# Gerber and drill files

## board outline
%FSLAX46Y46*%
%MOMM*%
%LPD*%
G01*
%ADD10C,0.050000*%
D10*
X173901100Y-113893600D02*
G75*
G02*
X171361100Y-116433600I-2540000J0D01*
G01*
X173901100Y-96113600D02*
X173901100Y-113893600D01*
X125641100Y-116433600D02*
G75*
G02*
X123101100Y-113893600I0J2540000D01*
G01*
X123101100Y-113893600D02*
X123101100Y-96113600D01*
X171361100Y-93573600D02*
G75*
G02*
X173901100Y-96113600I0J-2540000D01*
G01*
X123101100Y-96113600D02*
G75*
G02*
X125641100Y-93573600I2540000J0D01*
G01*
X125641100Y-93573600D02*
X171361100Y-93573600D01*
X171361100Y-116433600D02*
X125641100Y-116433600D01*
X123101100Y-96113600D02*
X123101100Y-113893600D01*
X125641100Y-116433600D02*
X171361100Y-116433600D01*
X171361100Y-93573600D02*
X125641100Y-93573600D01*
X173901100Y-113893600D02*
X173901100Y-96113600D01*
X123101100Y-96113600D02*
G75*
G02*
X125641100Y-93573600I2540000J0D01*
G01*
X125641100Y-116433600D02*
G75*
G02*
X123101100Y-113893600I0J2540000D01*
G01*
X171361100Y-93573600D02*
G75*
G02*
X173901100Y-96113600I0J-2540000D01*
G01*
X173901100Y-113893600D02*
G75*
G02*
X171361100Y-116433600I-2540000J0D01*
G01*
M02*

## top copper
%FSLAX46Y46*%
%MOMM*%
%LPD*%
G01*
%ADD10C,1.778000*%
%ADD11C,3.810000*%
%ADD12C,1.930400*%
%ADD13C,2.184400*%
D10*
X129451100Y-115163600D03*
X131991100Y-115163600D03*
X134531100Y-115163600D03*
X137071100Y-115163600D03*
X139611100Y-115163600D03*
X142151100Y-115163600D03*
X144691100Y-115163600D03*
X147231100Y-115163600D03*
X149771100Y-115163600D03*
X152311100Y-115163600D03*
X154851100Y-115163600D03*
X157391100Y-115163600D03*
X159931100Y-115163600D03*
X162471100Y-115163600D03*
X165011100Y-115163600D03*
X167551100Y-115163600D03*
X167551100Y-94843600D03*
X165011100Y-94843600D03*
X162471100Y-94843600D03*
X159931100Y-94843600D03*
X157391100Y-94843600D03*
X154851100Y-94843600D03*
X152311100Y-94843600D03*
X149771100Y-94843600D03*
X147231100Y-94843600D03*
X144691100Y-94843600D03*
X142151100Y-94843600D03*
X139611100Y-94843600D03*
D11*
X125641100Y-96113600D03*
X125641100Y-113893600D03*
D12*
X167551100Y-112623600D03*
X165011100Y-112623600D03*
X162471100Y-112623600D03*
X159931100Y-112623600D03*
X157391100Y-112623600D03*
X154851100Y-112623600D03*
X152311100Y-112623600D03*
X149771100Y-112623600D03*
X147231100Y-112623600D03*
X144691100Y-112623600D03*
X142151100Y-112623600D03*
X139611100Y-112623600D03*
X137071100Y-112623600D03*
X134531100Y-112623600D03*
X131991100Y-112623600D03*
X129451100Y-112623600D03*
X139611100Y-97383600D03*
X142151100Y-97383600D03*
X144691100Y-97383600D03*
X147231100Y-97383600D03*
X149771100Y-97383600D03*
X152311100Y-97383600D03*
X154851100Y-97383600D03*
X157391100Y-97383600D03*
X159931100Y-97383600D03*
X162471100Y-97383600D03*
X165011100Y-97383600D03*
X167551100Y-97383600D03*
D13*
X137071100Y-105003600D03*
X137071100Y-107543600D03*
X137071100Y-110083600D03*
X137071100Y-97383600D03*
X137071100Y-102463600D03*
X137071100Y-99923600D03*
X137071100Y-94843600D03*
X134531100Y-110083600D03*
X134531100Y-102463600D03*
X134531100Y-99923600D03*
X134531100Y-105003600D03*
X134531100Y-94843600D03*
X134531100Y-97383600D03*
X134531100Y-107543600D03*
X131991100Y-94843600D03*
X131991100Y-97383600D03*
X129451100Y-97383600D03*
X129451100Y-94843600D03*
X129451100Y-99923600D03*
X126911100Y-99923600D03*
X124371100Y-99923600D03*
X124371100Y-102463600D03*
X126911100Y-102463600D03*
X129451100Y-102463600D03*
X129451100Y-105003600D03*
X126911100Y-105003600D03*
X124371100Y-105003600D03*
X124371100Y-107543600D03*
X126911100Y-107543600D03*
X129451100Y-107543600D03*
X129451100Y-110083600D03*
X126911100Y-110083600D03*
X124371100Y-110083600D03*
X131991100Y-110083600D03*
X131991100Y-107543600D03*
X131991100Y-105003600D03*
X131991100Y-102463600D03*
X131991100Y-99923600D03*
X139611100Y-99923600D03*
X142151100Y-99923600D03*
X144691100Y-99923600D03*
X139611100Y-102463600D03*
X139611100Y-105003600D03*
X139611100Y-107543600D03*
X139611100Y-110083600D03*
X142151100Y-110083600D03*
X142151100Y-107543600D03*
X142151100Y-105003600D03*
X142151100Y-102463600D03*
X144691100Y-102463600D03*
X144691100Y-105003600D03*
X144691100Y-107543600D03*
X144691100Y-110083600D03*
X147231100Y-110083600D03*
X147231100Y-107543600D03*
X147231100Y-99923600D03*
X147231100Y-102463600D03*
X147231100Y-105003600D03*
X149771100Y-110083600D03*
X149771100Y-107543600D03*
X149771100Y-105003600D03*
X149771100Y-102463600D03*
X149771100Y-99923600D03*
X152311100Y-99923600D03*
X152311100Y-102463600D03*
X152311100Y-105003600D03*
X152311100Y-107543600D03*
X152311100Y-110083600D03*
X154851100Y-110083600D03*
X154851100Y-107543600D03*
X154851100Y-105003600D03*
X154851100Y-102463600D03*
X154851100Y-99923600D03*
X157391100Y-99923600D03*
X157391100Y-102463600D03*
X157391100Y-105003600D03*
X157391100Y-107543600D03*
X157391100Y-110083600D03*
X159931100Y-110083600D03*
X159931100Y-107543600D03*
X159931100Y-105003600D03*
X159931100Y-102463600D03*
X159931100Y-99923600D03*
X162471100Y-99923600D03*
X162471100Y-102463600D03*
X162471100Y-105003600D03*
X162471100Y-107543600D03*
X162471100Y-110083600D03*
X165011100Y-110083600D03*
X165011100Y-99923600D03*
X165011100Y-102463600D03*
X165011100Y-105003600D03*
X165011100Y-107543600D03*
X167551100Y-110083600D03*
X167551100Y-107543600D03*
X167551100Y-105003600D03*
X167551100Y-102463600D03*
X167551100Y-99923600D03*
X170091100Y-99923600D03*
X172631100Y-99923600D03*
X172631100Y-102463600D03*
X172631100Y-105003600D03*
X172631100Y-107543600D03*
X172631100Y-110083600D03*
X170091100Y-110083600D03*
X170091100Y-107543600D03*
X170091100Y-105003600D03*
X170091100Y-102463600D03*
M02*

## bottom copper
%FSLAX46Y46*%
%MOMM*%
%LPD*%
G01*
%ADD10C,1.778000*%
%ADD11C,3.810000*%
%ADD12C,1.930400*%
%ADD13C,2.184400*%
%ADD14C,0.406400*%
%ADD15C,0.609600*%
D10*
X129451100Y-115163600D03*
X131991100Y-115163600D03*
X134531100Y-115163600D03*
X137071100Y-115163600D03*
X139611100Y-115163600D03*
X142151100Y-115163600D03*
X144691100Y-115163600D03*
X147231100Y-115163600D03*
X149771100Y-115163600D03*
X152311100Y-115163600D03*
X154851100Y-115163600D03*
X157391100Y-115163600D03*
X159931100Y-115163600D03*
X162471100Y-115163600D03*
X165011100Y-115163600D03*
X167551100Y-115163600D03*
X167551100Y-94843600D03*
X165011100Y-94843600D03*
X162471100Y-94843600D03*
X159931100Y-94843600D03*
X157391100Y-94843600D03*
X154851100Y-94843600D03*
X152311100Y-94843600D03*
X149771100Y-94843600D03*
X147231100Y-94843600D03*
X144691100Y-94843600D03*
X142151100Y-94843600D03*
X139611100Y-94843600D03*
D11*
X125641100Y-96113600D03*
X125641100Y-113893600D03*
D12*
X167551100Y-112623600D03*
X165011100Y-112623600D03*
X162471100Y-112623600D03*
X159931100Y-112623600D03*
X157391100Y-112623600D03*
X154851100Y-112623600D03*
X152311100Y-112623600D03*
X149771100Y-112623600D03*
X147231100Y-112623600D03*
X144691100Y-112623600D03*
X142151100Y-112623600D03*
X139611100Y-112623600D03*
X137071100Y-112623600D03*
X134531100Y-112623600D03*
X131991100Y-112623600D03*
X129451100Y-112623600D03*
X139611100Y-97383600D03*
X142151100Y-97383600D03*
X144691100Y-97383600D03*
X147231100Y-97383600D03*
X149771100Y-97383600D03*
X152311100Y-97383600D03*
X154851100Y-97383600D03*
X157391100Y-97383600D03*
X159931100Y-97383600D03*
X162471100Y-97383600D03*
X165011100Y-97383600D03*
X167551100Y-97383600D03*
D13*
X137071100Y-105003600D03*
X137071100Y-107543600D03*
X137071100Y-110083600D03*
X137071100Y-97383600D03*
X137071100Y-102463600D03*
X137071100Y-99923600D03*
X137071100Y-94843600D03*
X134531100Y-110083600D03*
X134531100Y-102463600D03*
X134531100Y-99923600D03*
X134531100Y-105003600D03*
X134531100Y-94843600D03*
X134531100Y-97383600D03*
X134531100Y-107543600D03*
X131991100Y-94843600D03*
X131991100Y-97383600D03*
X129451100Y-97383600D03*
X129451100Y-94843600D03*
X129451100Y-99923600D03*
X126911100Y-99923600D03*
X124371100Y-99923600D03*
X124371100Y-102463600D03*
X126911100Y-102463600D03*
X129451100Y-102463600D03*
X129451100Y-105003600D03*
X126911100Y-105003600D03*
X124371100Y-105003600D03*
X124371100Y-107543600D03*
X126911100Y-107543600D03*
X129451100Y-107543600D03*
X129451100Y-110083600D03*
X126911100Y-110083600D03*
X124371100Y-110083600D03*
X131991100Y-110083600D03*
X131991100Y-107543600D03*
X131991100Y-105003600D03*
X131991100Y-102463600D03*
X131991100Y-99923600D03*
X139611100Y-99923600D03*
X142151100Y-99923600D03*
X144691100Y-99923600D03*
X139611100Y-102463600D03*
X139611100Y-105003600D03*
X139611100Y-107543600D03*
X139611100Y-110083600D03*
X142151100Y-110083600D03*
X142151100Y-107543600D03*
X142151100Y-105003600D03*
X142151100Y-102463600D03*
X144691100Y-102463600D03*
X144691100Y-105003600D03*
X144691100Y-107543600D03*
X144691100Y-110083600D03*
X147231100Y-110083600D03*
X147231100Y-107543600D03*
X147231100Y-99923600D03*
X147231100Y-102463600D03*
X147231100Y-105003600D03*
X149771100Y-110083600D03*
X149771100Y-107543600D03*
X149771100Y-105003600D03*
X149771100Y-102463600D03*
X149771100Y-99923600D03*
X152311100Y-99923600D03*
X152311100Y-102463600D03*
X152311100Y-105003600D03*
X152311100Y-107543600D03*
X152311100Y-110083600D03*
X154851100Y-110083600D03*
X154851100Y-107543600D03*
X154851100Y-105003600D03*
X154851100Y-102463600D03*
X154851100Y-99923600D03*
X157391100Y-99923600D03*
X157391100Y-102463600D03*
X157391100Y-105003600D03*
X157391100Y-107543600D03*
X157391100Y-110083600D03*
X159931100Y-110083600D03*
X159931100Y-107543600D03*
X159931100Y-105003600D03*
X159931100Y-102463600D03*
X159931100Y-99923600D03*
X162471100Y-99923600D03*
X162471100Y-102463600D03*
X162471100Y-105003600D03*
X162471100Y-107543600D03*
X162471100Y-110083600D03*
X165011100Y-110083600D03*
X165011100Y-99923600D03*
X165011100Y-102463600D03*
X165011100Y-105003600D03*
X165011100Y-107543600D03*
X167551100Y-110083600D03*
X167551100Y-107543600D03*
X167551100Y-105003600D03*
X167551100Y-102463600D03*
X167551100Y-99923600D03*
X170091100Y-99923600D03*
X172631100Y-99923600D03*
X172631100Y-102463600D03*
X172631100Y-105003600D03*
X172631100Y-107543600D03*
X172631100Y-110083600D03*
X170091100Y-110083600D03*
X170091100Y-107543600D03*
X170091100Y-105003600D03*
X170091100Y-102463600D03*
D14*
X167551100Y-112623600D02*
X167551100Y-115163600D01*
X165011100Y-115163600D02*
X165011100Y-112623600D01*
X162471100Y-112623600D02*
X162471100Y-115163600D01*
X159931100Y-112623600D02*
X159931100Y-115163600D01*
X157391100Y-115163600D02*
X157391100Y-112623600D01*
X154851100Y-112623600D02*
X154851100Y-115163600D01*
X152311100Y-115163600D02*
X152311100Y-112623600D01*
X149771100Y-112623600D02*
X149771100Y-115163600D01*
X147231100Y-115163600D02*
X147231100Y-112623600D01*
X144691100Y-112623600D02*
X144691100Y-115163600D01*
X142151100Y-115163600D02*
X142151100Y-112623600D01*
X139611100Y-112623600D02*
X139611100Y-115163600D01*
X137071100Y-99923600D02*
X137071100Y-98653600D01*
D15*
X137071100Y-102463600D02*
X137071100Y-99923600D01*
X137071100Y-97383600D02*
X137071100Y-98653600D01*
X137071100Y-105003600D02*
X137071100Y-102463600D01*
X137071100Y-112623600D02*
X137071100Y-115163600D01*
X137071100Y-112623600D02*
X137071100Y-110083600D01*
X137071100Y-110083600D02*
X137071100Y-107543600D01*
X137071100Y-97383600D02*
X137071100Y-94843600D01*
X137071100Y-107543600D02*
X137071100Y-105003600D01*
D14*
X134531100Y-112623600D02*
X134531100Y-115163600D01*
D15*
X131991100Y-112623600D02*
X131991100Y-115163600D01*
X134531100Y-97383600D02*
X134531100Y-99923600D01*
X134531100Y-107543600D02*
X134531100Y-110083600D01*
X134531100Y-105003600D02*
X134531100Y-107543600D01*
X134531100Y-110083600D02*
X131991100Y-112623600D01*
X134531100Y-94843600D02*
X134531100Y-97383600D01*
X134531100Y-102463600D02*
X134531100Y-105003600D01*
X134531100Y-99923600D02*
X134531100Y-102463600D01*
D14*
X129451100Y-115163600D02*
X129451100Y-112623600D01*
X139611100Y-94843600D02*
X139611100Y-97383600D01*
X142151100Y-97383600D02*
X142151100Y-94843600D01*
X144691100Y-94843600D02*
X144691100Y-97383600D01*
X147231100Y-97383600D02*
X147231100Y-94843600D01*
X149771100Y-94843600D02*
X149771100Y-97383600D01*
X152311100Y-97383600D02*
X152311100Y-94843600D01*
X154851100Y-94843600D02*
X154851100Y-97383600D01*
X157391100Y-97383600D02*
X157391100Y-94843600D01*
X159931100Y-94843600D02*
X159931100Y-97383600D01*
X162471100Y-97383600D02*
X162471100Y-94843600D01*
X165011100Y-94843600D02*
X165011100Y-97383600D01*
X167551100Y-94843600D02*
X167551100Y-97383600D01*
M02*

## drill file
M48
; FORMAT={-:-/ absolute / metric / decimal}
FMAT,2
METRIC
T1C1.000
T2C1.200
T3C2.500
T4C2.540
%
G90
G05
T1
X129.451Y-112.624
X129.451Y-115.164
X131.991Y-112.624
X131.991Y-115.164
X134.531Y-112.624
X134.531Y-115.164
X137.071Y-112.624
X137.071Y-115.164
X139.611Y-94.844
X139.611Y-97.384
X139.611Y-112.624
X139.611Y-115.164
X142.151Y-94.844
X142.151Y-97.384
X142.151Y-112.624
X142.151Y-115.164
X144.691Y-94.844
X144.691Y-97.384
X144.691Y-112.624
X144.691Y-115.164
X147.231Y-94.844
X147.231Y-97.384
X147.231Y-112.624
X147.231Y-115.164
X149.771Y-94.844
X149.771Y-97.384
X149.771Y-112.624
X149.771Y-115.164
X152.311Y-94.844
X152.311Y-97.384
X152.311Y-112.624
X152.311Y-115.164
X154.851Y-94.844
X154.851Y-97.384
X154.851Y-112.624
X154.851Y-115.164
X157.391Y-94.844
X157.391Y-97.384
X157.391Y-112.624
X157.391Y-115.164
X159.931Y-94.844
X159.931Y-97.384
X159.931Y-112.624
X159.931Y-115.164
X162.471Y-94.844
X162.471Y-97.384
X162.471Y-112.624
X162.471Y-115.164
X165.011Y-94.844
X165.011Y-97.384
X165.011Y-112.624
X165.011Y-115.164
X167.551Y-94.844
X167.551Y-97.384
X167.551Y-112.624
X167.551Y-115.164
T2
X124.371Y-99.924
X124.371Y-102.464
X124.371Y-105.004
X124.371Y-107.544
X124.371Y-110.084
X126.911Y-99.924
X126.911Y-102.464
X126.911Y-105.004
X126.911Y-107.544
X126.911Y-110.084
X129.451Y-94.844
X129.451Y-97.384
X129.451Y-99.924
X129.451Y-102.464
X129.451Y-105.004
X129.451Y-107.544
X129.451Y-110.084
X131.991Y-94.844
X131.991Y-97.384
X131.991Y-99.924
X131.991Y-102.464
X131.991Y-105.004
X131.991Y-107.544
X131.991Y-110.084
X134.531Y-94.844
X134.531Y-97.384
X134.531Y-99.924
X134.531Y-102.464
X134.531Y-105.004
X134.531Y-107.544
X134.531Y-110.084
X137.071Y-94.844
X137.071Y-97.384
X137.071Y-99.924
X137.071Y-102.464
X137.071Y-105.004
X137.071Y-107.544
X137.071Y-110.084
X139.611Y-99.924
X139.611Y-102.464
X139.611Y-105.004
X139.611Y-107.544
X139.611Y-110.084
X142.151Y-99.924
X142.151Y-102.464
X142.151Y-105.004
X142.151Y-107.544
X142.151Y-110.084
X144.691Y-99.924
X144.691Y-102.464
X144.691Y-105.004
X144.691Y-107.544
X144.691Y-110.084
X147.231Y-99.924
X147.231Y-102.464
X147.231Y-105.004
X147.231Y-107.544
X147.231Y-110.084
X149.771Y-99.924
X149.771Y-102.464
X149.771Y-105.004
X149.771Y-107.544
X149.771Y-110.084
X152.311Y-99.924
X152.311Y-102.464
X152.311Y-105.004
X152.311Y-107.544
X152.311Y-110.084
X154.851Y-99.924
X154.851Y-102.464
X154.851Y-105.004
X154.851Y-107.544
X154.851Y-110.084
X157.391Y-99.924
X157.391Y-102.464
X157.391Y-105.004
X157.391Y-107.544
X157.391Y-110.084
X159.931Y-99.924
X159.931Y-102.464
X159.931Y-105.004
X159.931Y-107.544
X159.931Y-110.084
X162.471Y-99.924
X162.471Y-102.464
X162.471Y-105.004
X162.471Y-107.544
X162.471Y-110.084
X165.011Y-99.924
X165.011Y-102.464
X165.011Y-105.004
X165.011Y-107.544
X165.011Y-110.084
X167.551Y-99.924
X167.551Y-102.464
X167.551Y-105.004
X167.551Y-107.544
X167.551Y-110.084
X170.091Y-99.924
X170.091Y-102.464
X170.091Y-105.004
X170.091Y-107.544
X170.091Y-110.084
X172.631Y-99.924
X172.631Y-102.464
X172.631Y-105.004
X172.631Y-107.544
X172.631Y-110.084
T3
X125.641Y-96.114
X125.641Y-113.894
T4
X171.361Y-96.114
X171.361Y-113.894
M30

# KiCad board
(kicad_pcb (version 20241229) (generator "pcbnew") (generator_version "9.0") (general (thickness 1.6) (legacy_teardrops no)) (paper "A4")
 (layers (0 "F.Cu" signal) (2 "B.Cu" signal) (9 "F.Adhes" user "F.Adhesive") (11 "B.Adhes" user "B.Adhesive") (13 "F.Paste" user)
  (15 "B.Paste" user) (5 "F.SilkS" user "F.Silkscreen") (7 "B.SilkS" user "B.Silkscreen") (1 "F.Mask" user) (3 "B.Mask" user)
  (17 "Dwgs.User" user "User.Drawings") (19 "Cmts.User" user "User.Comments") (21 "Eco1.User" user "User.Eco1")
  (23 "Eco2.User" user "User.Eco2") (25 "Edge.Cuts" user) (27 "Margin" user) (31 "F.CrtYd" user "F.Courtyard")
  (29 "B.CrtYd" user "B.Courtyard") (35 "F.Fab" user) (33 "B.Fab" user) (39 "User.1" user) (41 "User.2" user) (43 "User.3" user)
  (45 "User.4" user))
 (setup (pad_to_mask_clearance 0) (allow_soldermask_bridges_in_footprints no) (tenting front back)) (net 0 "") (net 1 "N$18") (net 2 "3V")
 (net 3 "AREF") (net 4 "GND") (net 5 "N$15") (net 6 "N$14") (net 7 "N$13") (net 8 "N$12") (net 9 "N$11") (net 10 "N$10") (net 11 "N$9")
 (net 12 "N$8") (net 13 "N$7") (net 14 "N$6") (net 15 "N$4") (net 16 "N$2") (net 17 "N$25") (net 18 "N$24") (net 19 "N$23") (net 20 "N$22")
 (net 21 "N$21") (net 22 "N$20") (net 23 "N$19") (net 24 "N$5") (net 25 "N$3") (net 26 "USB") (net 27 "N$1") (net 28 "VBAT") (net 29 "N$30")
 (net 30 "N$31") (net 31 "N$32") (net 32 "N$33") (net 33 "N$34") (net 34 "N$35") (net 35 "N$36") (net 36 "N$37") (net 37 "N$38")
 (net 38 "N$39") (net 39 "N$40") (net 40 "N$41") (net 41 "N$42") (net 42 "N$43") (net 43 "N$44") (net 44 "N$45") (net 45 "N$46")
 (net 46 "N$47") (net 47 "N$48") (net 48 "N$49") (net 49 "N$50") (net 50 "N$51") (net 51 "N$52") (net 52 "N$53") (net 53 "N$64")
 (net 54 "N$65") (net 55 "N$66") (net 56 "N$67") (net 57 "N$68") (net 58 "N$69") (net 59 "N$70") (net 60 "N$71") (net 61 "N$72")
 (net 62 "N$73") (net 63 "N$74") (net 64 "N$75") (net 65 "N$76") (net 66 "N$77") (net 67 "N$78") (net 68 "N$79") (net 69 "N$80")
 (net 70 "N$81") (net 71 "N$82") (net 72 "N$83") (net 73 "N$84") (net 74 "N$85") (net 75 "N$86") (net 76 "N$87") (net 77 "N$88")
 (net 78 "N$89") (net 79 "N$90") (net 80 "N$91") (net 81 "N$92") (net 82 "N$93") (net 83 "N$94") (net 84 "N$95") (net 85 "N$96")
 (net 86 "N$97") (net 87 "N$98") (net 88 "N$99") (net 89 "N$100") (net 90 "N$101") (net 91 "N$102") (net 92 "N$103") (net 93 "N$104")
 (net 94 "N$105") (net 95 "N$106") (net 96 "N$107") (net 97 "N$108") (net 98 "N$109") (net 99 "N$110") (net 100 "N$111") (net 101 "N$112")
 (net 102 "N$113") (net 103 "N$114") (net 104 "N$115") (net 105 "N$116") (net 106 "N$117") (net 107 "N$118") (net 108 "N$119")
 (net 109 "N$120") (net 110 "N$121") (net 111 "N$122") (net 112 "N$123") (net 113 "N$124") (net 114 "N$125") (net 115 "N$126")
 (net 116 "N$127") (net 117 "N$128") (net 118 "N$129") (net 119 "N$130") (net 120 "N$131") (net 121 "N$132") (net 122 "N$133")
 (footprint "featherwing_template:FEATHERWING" (layer "F.Cu") (at 123.1011 116.4336)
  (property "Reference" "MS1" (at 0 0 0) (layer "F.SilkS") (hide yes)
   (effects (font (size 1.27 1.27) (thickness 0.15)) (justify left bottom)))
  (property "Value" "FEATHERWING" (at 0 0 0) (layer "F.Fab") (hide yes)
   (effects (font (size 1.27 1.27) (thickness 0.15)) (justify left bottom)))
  (fp_line (start 0 -20.32) (end 0 -2.54) (stroke (width 0.05) (type solid)) (layer "Edge.Cuts"))
  (fp_line (start 2.54 0) (end 48.26 0) (stroke (width 0.05) (type solid)) (layer "Edge.Cuts"))
  (fp_line (start 48.26 -22.86) (end 2.54 -22.86) (stroke (width 0.05) (type solid)) (layer "Edge.Cuts"))
  (fp_line (start 50.8 -2.54) (end 50.8 -20.32) (stroke (width 0.05) (type solid)) (layer "Edge.Cuts"))
  (fp_arc (start 0 -20.32) (mid 0.743949 -22.116051) (end 2.54 -22.86) (stroke (width 0.05) (type solid)) (layer "Edge.Cuts"))
  (fp_arc (start 2.54 0) (mid 0.743949 -0.743949) (end 0 -2.54) (stroke (width 0.05) (type solid)) (layer "Edge.Cuts"))
  (fp_arc (start 48.26 -22.86) (mid 50.056051 -22.116051) (end 50.8 -20.32) (stroke (width 0.05) (type solid)) (layer "Edge.Cuts"))
  (fp_arc (start 50.8 -2.54) (mid 50.056051 -0.743949) (end 48.26 0) (stroke (width 0.05) (type solid)) (layer "Edge.Cuts"))
  (pad "" np_thru_hole circle (at 48.26 -20.32) (size 2.54 2.54) (drill 2.54) (layers "*.Cu" "*.Mask"))
  (pad "" np_thru_hole circle (at 48.26 -2.54) (size 2.54 2.54) (drill 2.54) (layers "*.Cu" "*.Mask"))
  (pad "1" thru_hole circle (at 6.35 -1.27) (size 1.778 1.778) (drill 1) (layers "*.Cu" "*.Mask") (remove_unused_layers no) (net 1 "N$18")
   (solder_mask_margin 0.0508) (thermal_bridge_angle 0))
  (pad "2" thru_hole circle (at 8.89 -1.27) (size 1.778 1.778) (drill 1) (layers "*.Cu" "*.Mask") (remove_unused_layers no) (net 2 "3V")
   (solder_mask_margin 0.0508) (thermal_bridge_angle 0))
  (pad "3" thru_hole circle (at 11.43 -1.27) (size 1.778 1.778) (drill 1) (layers "*.Cu" "*.Mask") (remove_unused_layers no) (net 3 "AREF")
   (solder_mask_margin 0.0508) (thermal_bridge_angle 0))
  (pad "4" thru_hole circle (at 13.97 -1.27) (size 1.778 1.778) (drill 1) (layers "*.Cu" "*.Mask") (remove_unused_layers no) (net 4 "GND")
   (solder_mask_margin 0.0508) (thermal_bridge_angle 0))
  (pad "5" thru_hole circle (at 16.51 -1.27) (size 1.778 1.778) (drill 1) (layers "*.Cu" "*.Mask") (remove_unused_layers no) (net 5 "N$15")
   (solder_mask_margin 0.0508) (thermal_bridge_angle 0))
  (pad "6" thru_hole circle (at 19.05 -1.27) (size 1.778 1.778) (drill 1) (layers "*.Cu" "*.Mask") (remove_unused_layers no) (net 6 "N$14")
   (solder_mask_margin 0.0508) (thermal_bridge_angle 0))
  (pad "7" thru_hole circle (at 21.59 -1.27) (size 1.778 1.778) (drill 1) (layers "*.Cu" "*.Mask") (remove_unused_layers no) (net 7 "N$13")
   (solder_mask_margin 0.0508) (thermal_bridge_angle 0))
  (pad "8" thru_hole circle (at 24.13 -1.27) (size 1.778 1.778) (drill 1) (layers "*.Cu" "*.Mask") (remove_unused_layers no) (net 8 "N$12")
   (solder_mask_margin 0.0508) (thermal_bridge_angle 0))
  (pad "9" thru_hole circle (at 26.67 -1.27) (size 1.778 1.778) (drill 1) (layers "*.Cu" "*.Mask") (remove_unused_layers no) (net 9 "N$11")
   (solder_mask_margin 0.0508) (thermal_bridge_angle 0))
  (pad "10" thru_hole circle (at 29.21 -1.27) (size 1.778 1.778) (drill 1) (layers "*.Cu" "*.Mask") (remove_unused_layers no)
   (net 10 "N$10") (solder_mask_margin 0.0508) (thermal_bridge_angle 0))
  (pad "11" thru_hole circle (at 31.75 -1.27) (size 1.778 1.778) (drill 1) (layers "*.Cu" "*.Mask") (remove_unused_layers no) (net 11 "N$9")
   (solder_mask_margin 0.0508) (thermal_bridge_angle 0))
  (pad "12" thru_hole circle (at 34.29 -1.27) (size 1.778 1.778) (drill 1) (layers "*.Cu" "*.Mask") (remove_unused_layers no) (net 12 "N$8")
   (solder_mask_margin 0.0508) (thermal_bridge_angle 0))
  (pad "13" thru_hole circle (at 36.83 -1.27) (size 1.778 1.778) (drill 1) (layers "*.Cu" "*.Mask") (remove_unused_layers no) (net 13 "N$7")
   (solder_mask_margin 0.0508) (thermal_bridge_angle 0))
  (pad "14" thru_hole circle (at 39.37 -1.27) (size 1.778 1.778) (drill 1) (layers "*.Cu" "*.Mask") (remove_unused_layers no) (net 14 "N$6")
   (solder_mask_margin 0.0508) (thermal_bridge_angle 0))
  (pad "15" thru_hole circle (at 41.91 -1.27) (size 1.778 1.778) (drill 1) (layers "*.Cu" "*.Mask") (remove_unused_layers no) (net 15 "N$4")
   (solder_mask_margin 0.0508) (thermal_bridge_angle 0))
  (pad "16" thru_hole circle (at 44.45 -1.27) (size 1.778 1.778) (drill 1) (layers "*.Cu" "*.Mask") (remove_unused_layers no) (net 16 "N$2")
   (solder_mask_margin 0.0508) (thermal_bridge_angle 0))
  (pad "17" thru_hole circle (at 44.45 -21.59) (size 1.778 1.778) (drill 1) (layers "*.Cu" "*.Mask") (remove_unused_layers no)
   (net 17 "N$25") (solder_mask_margin 0.0508) (thermal_bridge_angle 0))
  (pad "18" thru_hole circle (at 41.91 -21.59) (size 1.778 1.778) (drill 1) (layers "*.Cu" "*.Mask") (remove_unused_layers no)
   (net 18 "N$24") (solder_mask_margin 0.0508) (thermal_bridge_angle 0))
  (pad "19" thru_hole circle (at 39.37 -21.59) (size 1.778 1.778) (drill 1) (layers "*.Cu" "*.Mask") (remove_unused_layers no)
   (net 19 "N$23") (solder_mask_margin 0.0508) (thermal_bridge_angle 0))
  (pad "20" thru_hole circle (at 36.83 -21.59) (size 1.778 1.778) (drill 1) (layers "*.Cu" "*.Mask") (remove_unused_layers no)
   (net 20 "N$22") (solder_mask_margin 0.0508) (thermal_bridge_angle 0))
  (pad "21" thru_hole circle (at 34.29 -21.59) (size 1.778 1.778) (drill 1) (layers "*.Cu" "*.Mask") (remove_unused_layers no)
   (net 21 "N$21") (solder_mask_margin 0.0508) (thermal_bridge_angle 0))
  (pad "22" thru_hole circle (at 31.75 -21.59) (size 1.778 1.778) (drill 1) (layers "*.Cu" "*.Mask") (remove_unused_layers no)
   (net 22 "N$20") (solder_mask_margin 0.0508) (thermal_bridge_angle 0))
  (pad "23" thru_hole circle (at 29.21 -21.59) (size 1.778 1.778) (drill 1) (layers "*.Cu" "*.Mask") (remove_unused_layers no)
   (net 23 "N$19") (solder_mask_margin 0.0508) (thermal_bridge_angle 0))
  (pad "24" thru_hole circle (at 26.67 -21.59) (size 1.778 1.778) (drill 1) (layers "*.Cu" "*.Mask") (remove_unused_layers no)
   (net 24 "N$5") (solder_mask_margin 0.0508) (thermal_bridge_angle 0))
  (pad "25" thru_hole circle (at 24.13 -21.59) (size 1.778 1.778) (drill 1) (layers "*.Cu" "*.Mask") (remove_unused_layers no)
   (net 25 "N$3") (solder_mask_margin 0.0508) (thermal_bridge_angle 0))
  (pad "26" thru_hole circle (at 21.59 -21.59) (size 1.778 1.778) (drill 1) (layers "*.Cu" "*.Mask") (remove_unused_layers no)
   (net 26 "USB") (solder_mask_margin 0.0508) (thermal_bridge_angle 0))
  (pad "27" thru_hole circle (at 19.05 -21.59) (size 1.778 1.778) (drill 1) (layers "*.Cu" "*.Mask") (remove_unused_layers no)
   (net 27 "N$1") (solder_mask_margin 0.0508) (thermal_bridge_angle 0))
  (pad "28" thru_hole circle (at 16.51 -21.59) (size 1.778 1.778) (drill 1) (layers "*.Cu" "*.Mask") (remove_unused_layers no)
   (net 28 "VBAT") (solder_mask_margin 0.0508) (thermal_bridge_angle 0))
  (pad "P$1" thru_hole circle (at 2.54 -20.32) (size 3.81 3.81) (drill 2.5) (layers "*.Cu" "*.Mask") (remove_unused_layers no)
   (solder_mask_margin 0.0508) (thermal_bridge_angle 0))
  (pad "P$2" thru_hole circle (at 2.54 -2.54) (size 3.81 3.81) (drill 2.5) (layers "*.Cu" "*.Mask") (remove_unused_layers no)
   (solder_mask_margin 0.0508) (thermal_bridge_angle 0)))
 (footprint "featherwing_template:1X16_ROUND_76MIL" (layer "F.Cu") (at 148.5011 112.6236 180)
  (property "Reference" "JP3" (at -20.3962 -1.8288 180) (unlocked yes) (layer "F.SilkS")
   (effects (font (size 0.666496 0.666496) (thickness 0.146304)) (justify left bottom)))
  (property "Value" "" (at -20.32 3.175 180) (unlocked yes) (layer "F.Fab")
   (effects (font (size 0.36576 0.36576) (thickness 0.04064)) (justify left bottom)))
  (pad "1" thru_hole circle (at -19.05 0 270) (size 1.9304 1.9304) (drill 1) (layers "*.Cu" "*.Mask") (remove_unused_layers no)
   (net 16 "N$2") (solder_mask_margin 0.0508) (thermal_bridge_angle 0))
  (pad "2" thru_hole circle (at -16.51 0 270) (size 1.9304 1.9304) (drill 1) (layers "*.Cu" "*.Mask") (remove_unused_layers no)
   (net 15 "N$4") (solder_mask_margin 0.0508) (thermal_bridge_angle 0))
  (pad "3" thru_hole circle (at -13.97 0 270) (size 1.9304 1.9304) (drill 1) (layers "*.Cu" "*.Mask") (remove_unused_layers no)
   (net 14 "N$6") (solder_mask_margin 0.0508) (thermal_bridge_angle 0))
  (pad "4" thru_hole circle (at -11.43 0 270) (size 1.9304 1.9304) (drill 1) (layers "*.Cu" "*.Mask") (remove_unused_layers no)
   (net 13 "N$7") (solder_mask_margin 0.0508) (thermal_bridge_angle 0))
  (pad "5" thru_hole circle (at -8.89 0 270) (size 1.9304 1.9304) (drill 1) (layers "*.Cu" "*.Mask") (remove_unused_layers no)
   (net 12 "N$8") (solder_mask_margin 0.0508) (thermal_bridge_angle 0))
  (pad "6" thru_hole circle (at -6.35 0 270) (size 1.9304 1.9304) (drill 1) (layers "*.Cu" "*.Mask") (remove_unused_layers no)
   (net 11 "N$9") (solder_mask_margin 0.0508) (thermal_bridge_angle 0))
  (pad "7" thru_hole circle (at -3.81 0 270) (size 1.9304 1.9304) (drill 1) (layers "*.Cu" "*.Mask") (remove_unused_layers no)
   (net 10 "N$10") (solder_mask_margin 0.0508) (thermal_bridge_angle 0))
  (pad "8" thru_hole circle (at -1.27 0 270) (size 1.9304 1.9304) (drill 1) (layers "*.Cu" "*.Mask") (remove_unused_layers no)
   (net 9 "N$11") (solder_mask_margin 0.0508) (thermal_bridge_angle 0))
  (pad "9" thru_hole circle (at 1.27 0 270) (size 1.9304 1.9304) (drill 1) (layers "*.Cu" "*.Mask") (remove_unused_layers no) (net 8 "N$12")
   (solder_mask_margin 0.0508) (thermal_bridge_angle 0))
  (pad "10" thru_hole circle (at 3.81 0 270) (size 1.9304 1.9304) (drill 1) (layers "*.Cu" "*.Mask") (remove_unused_layers no)
   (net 7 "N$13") (solder_mask_margin 0.0508) (thermal_bridge_angle 0))
  (pad "11" thru_hole circle (at 6.35 0 270) (size 1.9304 1.9304) (drill 1) (layers "*.Cu" "*.Mask") (remove_unused_layers no)
   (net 6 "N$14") (solder_mask_margin 0.0508) (thermal_bridge_angle 0))
  (pad "12" thru_hole circle (at 8.89 0 270) (size 1.9304 1.9304) (drill 1) (layers "*.Cu" "*.Mask") (remove_unused_layers no)
   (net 5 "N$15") (solder_mask_margin 0.0508) (thermal_bridge_angle 0))
  (pad "13" thru_hole circle (at 11.43 0 270) (size 1.9304 1.9304) (drill 1) (layers "*.Cu" "*.Mask") (remove_unused_layers no)
   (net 4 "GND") (solder_mask_margin 0.0508) (thermal_bridge_angle 0))
  (pad "14" thru_hole circle (at 13.97 0 270) (size 1.9304 1.9304) (drill 1) (layers "*.Cu" "*.Mask") (remove_unused_layers no)
   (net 3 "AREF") (solder_mask_margin 0.0508) (thermal_bridge_angle 0))
  (pad "15" thru_hole circle (at 16.51 0 270) (size 1.9304 1.9304) (drill 1) (layers "*.Cu" "*.Mask") (remove_unused_layers no) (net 2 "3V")
   (solder_mask_margin 0.0508) (thermal_bridge_angle 0))
  (pad "16" thru_hole circle (at 19.05 0 270) (size 1.9304 1.9304) (drill 1) (layers "*.Cu" "*.Mask") (remove_unused_layers no)
   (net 1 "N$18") (solder_mask_margin 0.0508) (thermal_bridge_angle 0)))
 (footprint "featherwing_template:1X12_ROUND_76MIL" (layer "F.Cu") (at 153.5811 97.3836)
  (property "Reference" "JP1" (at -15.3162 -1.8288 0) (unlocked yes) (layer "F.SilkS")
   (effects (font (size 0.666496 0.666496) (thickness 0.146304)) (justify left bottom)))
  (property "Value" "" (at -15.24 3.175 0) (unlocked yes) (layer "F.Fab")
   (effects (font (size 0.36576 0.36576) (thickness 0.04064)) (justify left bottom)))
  (pad "1" thru_hole circle (at -13.97 0 90) (size 1.9304 1.9304) (drill 1) (layers "*.Cu" "*.Mask") (remove_unused_layers no)
   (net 28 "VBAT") (solder_mask_margin 0.0508) (thermal_bridge_angle 0))
  (pad "2" thru_hole circle (at -11.43 0 90) (size 1.9304 1.9304) (drill 1) (layers "*.Cu" "*.Mask") (remove_unused_layers no)
   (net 27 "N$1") (solder_mask_margin 0.0508) (thermal_bridge_angle 0))
  (pad "3" thru_hole circle (at -8.89 0 90) (size 1.9304 1.9304) (drill 1) (layers "*.Cu" "*.Mask") (remove_unused_layers no) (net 26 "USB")
   (solder_mask_margin 0.0508) (thermal_bridge_angle 0))
  (pad "4" thru_hole circle (at -6.35 0 90) (size 1.9304 1.9304) (drill 1) (layers "*.Cu" "*.Mask") (remove_unused_layers no) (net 25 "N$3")
   (solder_mask_margin 0.0508) (thermal_bridge_angle 0))
  (pad "5" thru_hole circle (at -3.81 0 90) (size 1.9304 1.9304) (drill 1) (layers "*.Cu" "*.Mask") (remove_unused_layers no) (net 24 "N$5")
   (solder_mask_margin 0.0508) (thermal_bridge_angle 0))
  (pad "6" thru_hole circle (at -1.27 0 90) (size 1.9304 1.9304) (drill 1) (layers "*.Cu" "*.Mask") (remove_unused_layers no)
   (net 23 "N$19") (solder_mask_margin 0.0508) (thermal_bridge_angle 0))
  (pad "7" thru_hole circle (at 1.27 0 90) (size 1.9304 1.9304) (drill 1) (layers "*.Cu" "*.Mask") (remove_unused_layers no) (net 22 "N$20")
   (solder_mask_margin 0.0508) (thermal_bridge_angle 0))
  (pad "8" thru_hole circle (at 3.81 0 90) (size 1.9304 1.9304) (drill 1) (layers "*.Cu" "*.Mask") (remove_unused_layers no) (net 21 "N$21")
   (solder_mask_margin 0.0508) (thermal_bridge_angle 0))
  (pad "9" thru_hole circle (at 6.35 0 90) (size 1.9304 1.9304) (drill 1) (layers "*.Cu" "*.Mask") (remove_unused_layers no) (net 20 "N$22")
   (solder_mask_margin 0.0508) (thermal_bridge_angle 0))
  (pad "10" thru_hole circle (at 8.89 0 90) (size 1.9304 1.9304) (drill 1) (layers "*.Cu" "*.Mask") (remove_unused_layers no)
   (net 19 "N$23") (solder_mask_margin 0.0508) (thermal_bridge_angle 0))
  (pad "11" thru_hole circle (at 11.43 0 90) (size 1.9304 1.9304) (drill 1) (layers "*.Cu" "*.Mask") (remove_unused_layers no)
   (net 18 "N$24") (solder_mask_margin 0.0508) (thermal_bridge_angle 0))
  (pad "12" thru_hole circle (at 13.97 0 90) (size 1.9304 1.9304) (drill 1) (layers "*.Cu" "*.Mask") (remove_unused_layers no)
   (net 17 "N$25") (solder_mask_margin 0.0508) (thermal_bridge_angle 0)))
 (gr_arc (start 173.9011 113.8936) (mid 173.157151 115.689651) (end 171.3611 116.4336) (stroke (width 0.05) (type solid))
  (layer "Edge.Cuts"))
 (gr_line (start 173.9011 96.1136) (end 173.9011 113.8936) (stroke (width 0.05) (type solid)) (layer "Edge.Cuts"))
 (gr_arc (start 125.6411 116.4336) (mid 123.845049 115.689651) (end 123.1011 113.8936) (stroke (width 0.05) (type solid))
  (layer "Edge.Cuts"))
 (gr_line (start 123.1011 113.8936) (end 123.1011 96.1136) (stroke (width 0.05) (type solid)) (layer "Edge.Cuts"))
 (gr_arc (start 171.3611 93.5736) (mid 173.157151 94.317549) (end 173.9011 96.1136) (stroke (width 0.05) (type solid)) (layer "Edge.Cuts"))
 (gr_arc (start 123.1011 96.1136) (mid 123.845049 94.317549) (end 125.6411 93.5736) (stroke (width 0.05) (type solid)) (layer "Edge.Cuts"))
 (gr_line (start 125.6411 93.5736) (end 171.3611 93.5736) (stroke (width 0.05) (type solid)) (layer "Edge.Cuts"))
 (gr_line (start 171.3611 116.4336) (end 125.6411 116.4336) (stroke (width 0.05) (type solid)) (layer "Edge.Cuts"))
 (segment (start 167.5511 112.6236) (end 167.5511 115.1636) (width 0.4064) (layer "B.Cu") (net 16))
 (segment (start 165.0111 115.1636) (end 165.0111 112.6236) (width 0.4064) (layer "B.Cu") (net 15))
 (segment (start 162.4711 112.6236) (end 162.4711 115.1636) (width 0.4064) (layer "B.Cu") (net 14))
 (segment (start 159.9311 112.6236) (end 159.9311 115.1636) (width 0.4064) (layer "B.Cu") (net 13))
 (segment (start 157.3911 115.1636) (end 157.3911 112.6236) (width 0.4064) (layer "B.Cu") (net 12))
 (segment (start 154.8511 112.6236) (end 154.8511 115.1636) (width 0.4064) (layer "B.Cu") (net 11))
 (segment (start 152.3111 115.1636) (end 152.3111 112.6236) (width 0.4064) (layer "B.Cu") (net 10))
 (segment (start 149.7711 112.6236) (end 149.7711 115.1636) (width 0.4064) (layer "B.Cu") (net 9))
 (segment (start 147.2311 115.1636) (end 147.2311 112.6236) (width 0.4064) (layer "B.Cu") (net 8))
 (segment (start 144.6911 112.6236) (end 144.6911 115.1636) (width 0.4064) (layer "B.Cu") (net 7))
 (segment (start 142.1511 115.1636) (end 142.1511 112.6236) (width 0.4064) (layer "B.Cu") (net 6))
 (segment (start 139.6111 112.6236) (end 139.6111 115.1636) (width 0.4064) (layer "B.Cu") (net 5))
 (via (at 137.0711 105.0036) (size 2.1844) (drill 1.2) (layers "F.Cu" "B.Cu") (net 4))
 (via (at 137.0711 107.5436) (size 2.1844) (drill 1.2) (layers "F.Cu" "B.Cu") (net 4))
 (via (at 137.0711 110.0836) (size 2.1844) (drill 1.2) (layers "F.Cu" "B.Cu") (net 4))
 (via (at 137.0711 97.3836) (size 2.1844) (drill 1.2) (layers "F.Cu" "B.Cu") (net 4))
 (via (at 137.0711 102.4636) (size 2.1844) (drill 1.2) (layers "F.Cu" "B.Cu") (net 4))
 (via (at 137.0711 99.9236) (size 2.1844) (drill 1.2) (layers "F.Cu" "B.Cu") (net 4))
 (via (at 137.0711 94.8436) (size 2.1844) (drill 1.2) (layers "F.Cu" "B.Cu") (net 4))
 (segment (start 137.0711 99.9236) (end 137.0711 98.6536) (width 0.4064) (layer "B.Cu") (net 4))
 (segment (start 137.0711 102.4636) (end 137.0711 99.9236) (width 0.6096) (layer "B.Cu") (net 4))
 (segment (start 137.0711 97.3836) (end 137.0711 98.6536) (width 0.6096) (layer "B.Cu") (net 4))
 (segment (start 137.0711 105.0036) (end 137.0711 102.4636) (width 0.6096) (layer "B.Cu") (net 4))
 (segment (start 137.0711 112.6236) (end 137.0711 115.1636) (width 0.6096) (layer "B.Cu") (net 4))
 (segment (start 137.0711 112.6236) (end 137.0711 110.0836) (width 0.6096) (layer "B.Cu") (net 4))
 (segment (start 137.0711 110.0836) (end 137.0711 107.5436) (width 0.6096) (layer "B.Cu") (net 4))
 (segment (start 137.0711 97.3836) (end 137.0711 94.8436) (width 0.6096) (layer "B.Cu") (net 4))
 (segment (start 137.0711 107.5436) (end 137.0711 105.0036) (width 0.6096) (layer "B.Cu") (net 4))
 (segment (start 134.5311 112.6236) (end 134.5311 115.1636) (width 0.4064) (layer "B.Cu") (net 3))
 (via (at 134.5311 110.0836) (size 2.1844) (drill 1.2) (layers "F.Cu" "B.Cu") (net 2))
 (via (at 134.5311 102.4636) (size 2.1844) (drill 1.2) (layers "F.Cu" "B.Cu") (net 2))
 (via (at 134.5311 99.9236) (size 2.1844) (drill 1.2) (layers "F.Cu" "B.Cu") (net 2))
 (via (at 134.5311 105.0036) (size 2.1844) (drill 1.2) (layers "F.Cu" "B.Cu") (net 2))
 (via (at 134.5311 94.8436) (size 2.1844) (drill 1.2) (layers "F.Cu" "B.Cu") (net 2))
 (via (at 134.5311 97.3836) (size 2.1844) (drill 1.2) (layers "F.Cu" "B.Cu") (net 2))
 (via (at 134.5311 107.5436) (size 2.1844) (drill 1.2) (layers "F.Cu" "B.Cu") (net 2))
 (segment (start 131.9911 112.6236) (end 131.9911 115.1636) (width 0.6096) (layer "B.Cu") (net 2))
 (segment (start 134.5311 97.3836) (end 134.5311 99.9236) (width 0.6096) (layer "B.Cu") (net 2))
 (segment (start 134.5311 107.5436) (end 134.5311 110.0836) (width 0.6096) (layer "B.Cu") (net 2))
 (segment (start 134.5311 105.0036) (end 134.5311 107.5436) (width 0.6096) (layer "B.Cu") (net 2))
 (segment (start 134.5311 110.0836) (end 131.9911 112.6236) (width 0.6096) (layer "B.Cu") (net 2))
 (segment (start 134.5311 94.8436) (end 134.5311 97.3836) (width 0.6096) (layer "B.Cu") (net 2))
 (segment (start 134.5311 102.4636) (end 134.5311 105.0036) (width 0.6096) (layer "B.Cu") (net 2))
 (segment (start 134.5311 99.9236) (end 134.5311 102.4636) (width 0.6096) (layer "B.Cu") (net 2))
 (segment (start 129.4511 115.1636) (end 129.4511 112.6236) (width 0.4064) (layer "B.Cu") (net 1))
 (segment (start 139.6111 94.8436) (end 139.6111 97.3836) (width 0.4064) (layer "B.Cu") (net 28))
 (segment (start 142.1511 97.3836) (end 142.1511 94.8436) (width 0.4064) (layer "B.Cu") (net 27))
 (segment (start 144.6911 94.8436) (end 144.6911 97.3836) (width 0.4064) (layer "B.Cu") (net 26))
 (segment (start 147.2311 97.3836) (end 147.2311 94.8436) (width 0.4064) (layer "B.Cu") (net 25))
 (segment (start 149.7711 94.8436) (end 149.7711 97.3836) (width 0.4064) (layer "B.Cu") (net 24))
 (segment (start 152.3111 97.3836) (end 152.3111 94.8436) (width 0.4064) (layer "B.Cu") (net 23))
 (segment (start 154.8511 94.8436) (end 154.8511 97.3836) (width 0.4064) (layer "B.Cu") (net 22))
 (segment (start 157.3911 97.3836) (end 157.3911 94.8436) (width 0.4064) (layer "B.Cu") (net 21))
 (segment (start 159.9311 94.8436) (end 159.9311 97.3836) (width 0.4064) (layer "B.Cu") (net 20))
 (segment (start 162.4711 97.3836) (end 162.4711 94.8436) (width 0.4064) (layer "B.Cu") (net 19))
 (segment (start 165.0111 94.8436) (end 165.0111 97.3836) (width 0.4064) (layer "B.Cu") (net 18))
 (segment (start 167.5511 94.8436) (end 167.5511 97.3836) (width 0.4064) (layer "B.Cu") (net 17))
 (via (at 131.9911 94.8436) (size 2.1844) (drill 1.2) (layers "F.Cu" "B.Cu") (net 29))
 (via (at 131.9911 97.3836) (size 2.1844) (drill 1.2) (layers "F.Cu" "B.Cu") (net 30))
 (via (at 129.4511 97.3836) (size 2.1844) (drill 1.2) (layers "F.Cu" "B.Cu") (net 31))
 (via (at 129.4511 94.8436) (size 2.1844) (drill 1.2) (layers "F.Cu" "B.Cu") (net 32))
 (via (at 129.4511 99.9236) (size 2.1844) (drill 1.2) (layers "F.Cu" "B.Cu") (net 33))
 (via (at 126.9111 99.9236) (size 2.1844) (drill 1.2) (layers "F.Cu" "B.Cu") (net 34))
 (via (at 124.3711 99.9236) (size 2.1844) (drill 1.2) (layers "F.Cu" "B.Cu") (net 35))
 (via (at 124.3711 102.4636) (size 2.1844) (drill 1.2) (layers "F.Cu" "B.Cu") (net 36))
 (via (at 126.9111 102.4636) (size 2.1844) (drill 1.2) (layers "F.Cu" "B.Cu") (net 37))
 (via (at 129.4511 102.4636) (size 2.1844) (drill 1.2) (layers "F.Cu" "B.Cu") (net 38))
 (via (at 129.4511 105.0036) (size 2.1844) (drill 1.2) (layers "F.Cu" "B.Cu") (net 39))
 (via (at 126.9111 105.0036) (size 2.1844) (drill 1.2) (layers "F.Cu" "B.Cu") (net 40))
 (via (at 124.3711 105.0036) (size 2.1844) (drill 1.2) (layers "F.Cu" "B.Cu") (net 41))
 (via (at 124.3711 107.5436) (size 2.1844) (drill 1.2) (layers "F.Cu" "B.Cu") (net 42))
 (via (at 126.9111 107.5436) (size 2.1844) (drill 1.2) (layers "F.Cu" "B.Cu") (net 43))
 (via (at 129.4511 107.5436) (size 2.1844) (drill 1.2) (layers "F.Cu" "B.Cu") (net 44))
 (via (at 129.4511 110.0836) (size 2.1844) (drill 1.2) (layers "F.Cu" "B.Cu") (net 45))
 (via (at 126.9111 110.0836) (size 2.1844) (drill 1.2) (layers "F.Cu" "B.Cu") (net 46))
 (via (at 124.3711 110.0836) (size 2.1844) (drill 1.2) (layers "F.Cu" "B.Cu") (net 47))
 (via (at 131.9911 110.0836) (size 2.1844) (drill 1.2) (layers "F.Cu" "B.Cu") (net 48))
 (via (at 131.9911 107.5436) (size 2.1844) (drill 1.2) (layers "F.Cu" "B.Cu") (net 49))
 (via (at 131.9911 105.0036) (size 2.1844) (drill 1.2) (layers "F.Cu" "B.Cu") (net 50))
 (via (at 131.9911 102.4636) (size 2.1844) (drill 1.2) (layers "F.Cu" "B.Cu") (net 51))
 (via (at 131.9911 99.9236) (size 2.1844) (drill 1.2) (layers "F.Cu" "B.Cu") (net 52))
 (via (at 139.6111 99.9236) (size 2.1844) (drill 1.2) (layers "F.Cu" "B.Cu") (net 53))
 (via (at 142.1511 99.9236) (size 2.1844) (drill 1.2) (layers "F.Cu" "B.Cu") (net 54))
 (via (at 144.6911 99.9236) (size 2.1844) (drill 1.2) (layers "F.Cu" "B.Cu") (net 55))
 (via (at 139.6111 102.4636) (size 2.1844) (drill 1.2) (layers "F.Cu" "B.Cu") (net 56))
 (via (at 139.6111 105.0036) (size 2.1844) (drill 1.2) (layers "F.Cu" "B.Cu") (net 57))
 (via (at 139.6111 107.5436) (size 2.1844) (drill 1.2) (layers "F.Cu" "B.Cu") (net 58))
 (via (at 139.6111 110.0836) (size 2.1844) (drill 1.2) (layers "F.Cu" "B.Cu") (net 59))
 (via (at 142.1511 110.0836) (size 2.1844) (drill 1.2) (layers "F.Cu" "B.Cu") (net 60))
 (via (at 142.1511 107.5436) (size 2.1844) (drill 1.2) (layers "F.Cu" "B.Cu") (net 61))
 (via (at 142.1511 105.0036) (size 2.1844) (drill 1.2) (layers "F.Cu" "B.Cu") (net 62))
 (via (at 142.1511 102.4636) (size 2.1844) (drill 1.2) (layers "F.Cu" "B.Cu") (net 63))
 (via (at 144.6911 102.4636) (size 2.1844) (drill 1.2) (layers "F.Cu" "B.Cu") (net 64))
 (via (at 144.6911 105.0036) (size 2.1844) (drill 1.2) (layers "F.Cu" "B.Cu") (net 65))
 (via (at 144.6911 107.5436) (size 2.1844) (drill 1.2) (layers "F.Cu" "B.Cu") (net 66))
 (via (at 144.6911 110.0836) (size 2.1844) (drill 1.2) (layers "F.Cu" "B.Cu") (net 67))
 (via (at 147.2311 110.0836) (size 2.1844) (drill 1.2) (layers "F.Cu" "B.Cu") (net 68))
 (via (at 147.2311 107.5436) (size 2.1844) (drill 1.2) (layers "F.Cu" "B.Cu") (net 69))
 (via (at 147.2311 99.9236) (size 2.1844) (drill 1.2) (layers "F.Cu" "B.Cu") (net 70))
 (via (at 147.2311 102.4636) (size 2.1844) (drill 1.2) (layers "F.Cu" "B.Cu") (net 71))
 (via (at 147.2311 105.0036) (size 2.1844) (drill 1.2) (layers "F.Cu" "B.Cu") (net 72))
 (via (at 149.7711 110.0836) (size 2.1844) (drill 1.2) (layers "F.Cu" "B.Cu") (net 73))
 (via (at 149.7711 107.5436) (size 2.1844) (drill 1.2) (layers "F.Cu" "B.Cu") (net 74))
 (via (at 149.7711 105.0036) (size 2.1844) (drill 1.2) (layers "F.Cu" "B.Cu") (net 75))
 (via (at 149.7711 102.4636) (size 2.1844) (drill 1.2) (layers "F.Cu" "B.Cu") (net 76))
 (via (at 149.7711 99.9236) (size 2.1844) (drill 1.2) (layers "F.Cu" "B.Cu") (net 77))
 (via (at 152.3111 99.9236) (size 2.1844) (drill 1.2) (layers "F.Cu" "B.Cu") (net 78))
 (via (at 152.3111 102.4636) (size 2.1844) (drill 1.2) (layers "F.Cu" "B.Cu") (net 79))
 (via (at 152.3111 105.0036) (size 2.1844) (drill 1.2) (layers "F.Cu" "B.Cu") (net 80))
 (via (at 152.3111 107.5436) (size 2.1844) (drill 1.2) (layers "F.Cu" "B.Cu") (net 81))
 (via (at 152.3111 110.0836) (size 2.1844) (drill 1.2) (layers "F.Cu" "B.Cu") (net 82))
 (via (at 154.8511 110.0836) (size 2.1844) (drill 1.2) (layers "F.Cu" "B.Cu") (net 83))
 (via (at 154.8511 107.5436) (size 2.1844) (drill 1.2) (layers "F.Cu" "B.Cu") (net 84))
 (via (at 154.8511 105.0036) (size 2.1844) (drill 1.2) (layers "F.Cu" "B.Cu") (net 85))
 (via (at 154.8511 102.4636) (size 2.1844) (drill 1.2) (layers "F.Cu" "B.Cu") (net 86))
 (via (at 154.8511 99.9236) (size 2.1844) (drill 1.2) (layers "F.Cu" "B.Cu") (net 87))
 (via (at 157.3911 99.9236) (size 2.1844) (drill 1.2) (layers "F.Cu" "B.Cu") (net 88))
 (via (at 157.3911 102.4636) (size 2.1844) (drill 1.2) (layers "F.Cu" "B.Cu") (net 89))
 (via (at 157.3911 105.0036) (size 2.1844) (drill 1.2) (layers "F.Cu" "B.Cu") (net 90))
 (via (at 157.3911 107.5436) (size 2.1844) (drill 1.2) (layers "F.Cu" "B.Cu") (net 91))
 (via (at 157.3911 110.0836) (size 2.1844) (drill 1.2) (layers "F.Cu" "B.Cu") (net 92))
 (via (at 159.9311 110.0836) (size 2.1844) (drill 1.2) (layers "F.Cu" "B.Cu") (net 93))
 (via (at 159.9311 107.5436) (size 2.1844) (drill 1.2) (layers "F.Cu" "B.Cu") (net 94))
 (via (at 159.9311 105.0036) (size 2.1844) (drill 1.2) (layers "F.Cu" "B.Cu") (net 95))
 (via (at 159.9311 102.4636) (size 2.1844) (drill 1.2) (layers "F.Cu" "B.Cu") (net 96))
 (via (at 159.9311 99.9236) (size 2.1844) (drill 1.2) (layers "F.Cu" "B.Cu") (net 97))
 (via (at 162.4711 99.9236) (size 2.1844) (drill 1.2) (layers "F.Cu" "B.Cu") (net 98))
 (via (at 162.4711 102.4636) (size 2.1844) (drill 1.2) (layers "F.Cu" "B.Cu") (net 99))
 (via (at 162.4711 105.0036) (size 2.1844) (drill 1.2) (layers "F.Cu" "B.Cu") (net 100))
 (via (at 162.4711 107.5436) (size 2.1844) (drill 1.2) (layers "F.Cu" "B.Cu") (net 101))
 (via (at 162.4711 110.0836) (size 2.1844) (drill 1.2) (layers "F.Cu" "B.Cu") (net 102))
 (via (at 165.0111 110.0836) (size 2.1844) (drill 1.2) (layers "F.Cu" "B.Cu") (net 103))
 (via (at 165.0111 99.9236) (size 2.1844) (drill 1.2) (layers "F.Cu" "B.Cu") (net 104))
 (via (at 165.0111 102.4636) (size 2.1844) (drill 1.2) (layers "F.Cu" "B.Cu") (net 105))
 (via (at 165.0111 105.0036) (size 2.1844) (drill 1.2) (layers "F.Cu" "B.Cu") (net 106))
 (via (at 165.0111 107.5436) (size 2.1844) (drill 1.2) (layers "F.Cu" "B.Cu") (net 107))
 (via (at 167.5511 110.0836) (size 2.1844) (drill 1.2) (layers "F.Cu" "B.Cu") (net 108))
 (via (at 167.5511 107.5436) (size 2.1844) (drill 1.2) (layers "F.Cu" "B.Cu") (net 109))
 (via (at 167.5511 105.0036) (size 2.1844) (drill 1.2) (layers "F.Cu" "B.Cu") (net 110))
 (via (at 167.5511 102.4636) (size 2.1844) (drill 1.2) (layers "F.Cu" "B.Cu") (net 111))
 (via (at 167.5511 99.9236) (size 2.1844) (drill 1.2) (layers "F.Cu" "B.Cu") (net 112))
 (via (at 170.0911 99.9236) (size 2.1844) (drill 1.2) (layers "F.Cu" "B.Cu") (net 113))
 (via (at 172.6311 99.9236) (size 2.1844) (drill 1.2) (layers "F.Cu" "B.Cu") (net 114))
 (via (at 172.6311 102.4636) (size 2.1844) (drill 1.2) (layers "F.Cu" "B.Cu") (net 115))
 (via (at 172.6311 105.0036) (size 2.1844) (drill 1.2) (layers "F.Cu" "B.Cu") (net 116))
 (via (at 172.6311 107.5436) (size 2.1844) (drill 1.2) (layers "F.Cu" "B.Cu") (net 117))
 (via (at 172.6311 110.0836) (size 2.1844) (drill 1.2) (layers "F.Cu" "B.Cu") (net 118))
 (via (at 170.0911 110.0836) (size 2.1844) (drill 1.2) (layers "F.Cu" "B.Cu") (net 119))
 (via (at 170.0911 107.5436) (size 2.1844) (drill 1.2) (layers "F.Cu" "B.Cu") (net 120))
 (via (at 170.0911 105.0036) (size 2.1844) (drill 1.2) (layers "F.Cu" "B.Cu") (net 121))
 (via (at 170.0911 102.4636) (size 2.1844) (drill 1.2) (layers "F.Cu" "B.Cu") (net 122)))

